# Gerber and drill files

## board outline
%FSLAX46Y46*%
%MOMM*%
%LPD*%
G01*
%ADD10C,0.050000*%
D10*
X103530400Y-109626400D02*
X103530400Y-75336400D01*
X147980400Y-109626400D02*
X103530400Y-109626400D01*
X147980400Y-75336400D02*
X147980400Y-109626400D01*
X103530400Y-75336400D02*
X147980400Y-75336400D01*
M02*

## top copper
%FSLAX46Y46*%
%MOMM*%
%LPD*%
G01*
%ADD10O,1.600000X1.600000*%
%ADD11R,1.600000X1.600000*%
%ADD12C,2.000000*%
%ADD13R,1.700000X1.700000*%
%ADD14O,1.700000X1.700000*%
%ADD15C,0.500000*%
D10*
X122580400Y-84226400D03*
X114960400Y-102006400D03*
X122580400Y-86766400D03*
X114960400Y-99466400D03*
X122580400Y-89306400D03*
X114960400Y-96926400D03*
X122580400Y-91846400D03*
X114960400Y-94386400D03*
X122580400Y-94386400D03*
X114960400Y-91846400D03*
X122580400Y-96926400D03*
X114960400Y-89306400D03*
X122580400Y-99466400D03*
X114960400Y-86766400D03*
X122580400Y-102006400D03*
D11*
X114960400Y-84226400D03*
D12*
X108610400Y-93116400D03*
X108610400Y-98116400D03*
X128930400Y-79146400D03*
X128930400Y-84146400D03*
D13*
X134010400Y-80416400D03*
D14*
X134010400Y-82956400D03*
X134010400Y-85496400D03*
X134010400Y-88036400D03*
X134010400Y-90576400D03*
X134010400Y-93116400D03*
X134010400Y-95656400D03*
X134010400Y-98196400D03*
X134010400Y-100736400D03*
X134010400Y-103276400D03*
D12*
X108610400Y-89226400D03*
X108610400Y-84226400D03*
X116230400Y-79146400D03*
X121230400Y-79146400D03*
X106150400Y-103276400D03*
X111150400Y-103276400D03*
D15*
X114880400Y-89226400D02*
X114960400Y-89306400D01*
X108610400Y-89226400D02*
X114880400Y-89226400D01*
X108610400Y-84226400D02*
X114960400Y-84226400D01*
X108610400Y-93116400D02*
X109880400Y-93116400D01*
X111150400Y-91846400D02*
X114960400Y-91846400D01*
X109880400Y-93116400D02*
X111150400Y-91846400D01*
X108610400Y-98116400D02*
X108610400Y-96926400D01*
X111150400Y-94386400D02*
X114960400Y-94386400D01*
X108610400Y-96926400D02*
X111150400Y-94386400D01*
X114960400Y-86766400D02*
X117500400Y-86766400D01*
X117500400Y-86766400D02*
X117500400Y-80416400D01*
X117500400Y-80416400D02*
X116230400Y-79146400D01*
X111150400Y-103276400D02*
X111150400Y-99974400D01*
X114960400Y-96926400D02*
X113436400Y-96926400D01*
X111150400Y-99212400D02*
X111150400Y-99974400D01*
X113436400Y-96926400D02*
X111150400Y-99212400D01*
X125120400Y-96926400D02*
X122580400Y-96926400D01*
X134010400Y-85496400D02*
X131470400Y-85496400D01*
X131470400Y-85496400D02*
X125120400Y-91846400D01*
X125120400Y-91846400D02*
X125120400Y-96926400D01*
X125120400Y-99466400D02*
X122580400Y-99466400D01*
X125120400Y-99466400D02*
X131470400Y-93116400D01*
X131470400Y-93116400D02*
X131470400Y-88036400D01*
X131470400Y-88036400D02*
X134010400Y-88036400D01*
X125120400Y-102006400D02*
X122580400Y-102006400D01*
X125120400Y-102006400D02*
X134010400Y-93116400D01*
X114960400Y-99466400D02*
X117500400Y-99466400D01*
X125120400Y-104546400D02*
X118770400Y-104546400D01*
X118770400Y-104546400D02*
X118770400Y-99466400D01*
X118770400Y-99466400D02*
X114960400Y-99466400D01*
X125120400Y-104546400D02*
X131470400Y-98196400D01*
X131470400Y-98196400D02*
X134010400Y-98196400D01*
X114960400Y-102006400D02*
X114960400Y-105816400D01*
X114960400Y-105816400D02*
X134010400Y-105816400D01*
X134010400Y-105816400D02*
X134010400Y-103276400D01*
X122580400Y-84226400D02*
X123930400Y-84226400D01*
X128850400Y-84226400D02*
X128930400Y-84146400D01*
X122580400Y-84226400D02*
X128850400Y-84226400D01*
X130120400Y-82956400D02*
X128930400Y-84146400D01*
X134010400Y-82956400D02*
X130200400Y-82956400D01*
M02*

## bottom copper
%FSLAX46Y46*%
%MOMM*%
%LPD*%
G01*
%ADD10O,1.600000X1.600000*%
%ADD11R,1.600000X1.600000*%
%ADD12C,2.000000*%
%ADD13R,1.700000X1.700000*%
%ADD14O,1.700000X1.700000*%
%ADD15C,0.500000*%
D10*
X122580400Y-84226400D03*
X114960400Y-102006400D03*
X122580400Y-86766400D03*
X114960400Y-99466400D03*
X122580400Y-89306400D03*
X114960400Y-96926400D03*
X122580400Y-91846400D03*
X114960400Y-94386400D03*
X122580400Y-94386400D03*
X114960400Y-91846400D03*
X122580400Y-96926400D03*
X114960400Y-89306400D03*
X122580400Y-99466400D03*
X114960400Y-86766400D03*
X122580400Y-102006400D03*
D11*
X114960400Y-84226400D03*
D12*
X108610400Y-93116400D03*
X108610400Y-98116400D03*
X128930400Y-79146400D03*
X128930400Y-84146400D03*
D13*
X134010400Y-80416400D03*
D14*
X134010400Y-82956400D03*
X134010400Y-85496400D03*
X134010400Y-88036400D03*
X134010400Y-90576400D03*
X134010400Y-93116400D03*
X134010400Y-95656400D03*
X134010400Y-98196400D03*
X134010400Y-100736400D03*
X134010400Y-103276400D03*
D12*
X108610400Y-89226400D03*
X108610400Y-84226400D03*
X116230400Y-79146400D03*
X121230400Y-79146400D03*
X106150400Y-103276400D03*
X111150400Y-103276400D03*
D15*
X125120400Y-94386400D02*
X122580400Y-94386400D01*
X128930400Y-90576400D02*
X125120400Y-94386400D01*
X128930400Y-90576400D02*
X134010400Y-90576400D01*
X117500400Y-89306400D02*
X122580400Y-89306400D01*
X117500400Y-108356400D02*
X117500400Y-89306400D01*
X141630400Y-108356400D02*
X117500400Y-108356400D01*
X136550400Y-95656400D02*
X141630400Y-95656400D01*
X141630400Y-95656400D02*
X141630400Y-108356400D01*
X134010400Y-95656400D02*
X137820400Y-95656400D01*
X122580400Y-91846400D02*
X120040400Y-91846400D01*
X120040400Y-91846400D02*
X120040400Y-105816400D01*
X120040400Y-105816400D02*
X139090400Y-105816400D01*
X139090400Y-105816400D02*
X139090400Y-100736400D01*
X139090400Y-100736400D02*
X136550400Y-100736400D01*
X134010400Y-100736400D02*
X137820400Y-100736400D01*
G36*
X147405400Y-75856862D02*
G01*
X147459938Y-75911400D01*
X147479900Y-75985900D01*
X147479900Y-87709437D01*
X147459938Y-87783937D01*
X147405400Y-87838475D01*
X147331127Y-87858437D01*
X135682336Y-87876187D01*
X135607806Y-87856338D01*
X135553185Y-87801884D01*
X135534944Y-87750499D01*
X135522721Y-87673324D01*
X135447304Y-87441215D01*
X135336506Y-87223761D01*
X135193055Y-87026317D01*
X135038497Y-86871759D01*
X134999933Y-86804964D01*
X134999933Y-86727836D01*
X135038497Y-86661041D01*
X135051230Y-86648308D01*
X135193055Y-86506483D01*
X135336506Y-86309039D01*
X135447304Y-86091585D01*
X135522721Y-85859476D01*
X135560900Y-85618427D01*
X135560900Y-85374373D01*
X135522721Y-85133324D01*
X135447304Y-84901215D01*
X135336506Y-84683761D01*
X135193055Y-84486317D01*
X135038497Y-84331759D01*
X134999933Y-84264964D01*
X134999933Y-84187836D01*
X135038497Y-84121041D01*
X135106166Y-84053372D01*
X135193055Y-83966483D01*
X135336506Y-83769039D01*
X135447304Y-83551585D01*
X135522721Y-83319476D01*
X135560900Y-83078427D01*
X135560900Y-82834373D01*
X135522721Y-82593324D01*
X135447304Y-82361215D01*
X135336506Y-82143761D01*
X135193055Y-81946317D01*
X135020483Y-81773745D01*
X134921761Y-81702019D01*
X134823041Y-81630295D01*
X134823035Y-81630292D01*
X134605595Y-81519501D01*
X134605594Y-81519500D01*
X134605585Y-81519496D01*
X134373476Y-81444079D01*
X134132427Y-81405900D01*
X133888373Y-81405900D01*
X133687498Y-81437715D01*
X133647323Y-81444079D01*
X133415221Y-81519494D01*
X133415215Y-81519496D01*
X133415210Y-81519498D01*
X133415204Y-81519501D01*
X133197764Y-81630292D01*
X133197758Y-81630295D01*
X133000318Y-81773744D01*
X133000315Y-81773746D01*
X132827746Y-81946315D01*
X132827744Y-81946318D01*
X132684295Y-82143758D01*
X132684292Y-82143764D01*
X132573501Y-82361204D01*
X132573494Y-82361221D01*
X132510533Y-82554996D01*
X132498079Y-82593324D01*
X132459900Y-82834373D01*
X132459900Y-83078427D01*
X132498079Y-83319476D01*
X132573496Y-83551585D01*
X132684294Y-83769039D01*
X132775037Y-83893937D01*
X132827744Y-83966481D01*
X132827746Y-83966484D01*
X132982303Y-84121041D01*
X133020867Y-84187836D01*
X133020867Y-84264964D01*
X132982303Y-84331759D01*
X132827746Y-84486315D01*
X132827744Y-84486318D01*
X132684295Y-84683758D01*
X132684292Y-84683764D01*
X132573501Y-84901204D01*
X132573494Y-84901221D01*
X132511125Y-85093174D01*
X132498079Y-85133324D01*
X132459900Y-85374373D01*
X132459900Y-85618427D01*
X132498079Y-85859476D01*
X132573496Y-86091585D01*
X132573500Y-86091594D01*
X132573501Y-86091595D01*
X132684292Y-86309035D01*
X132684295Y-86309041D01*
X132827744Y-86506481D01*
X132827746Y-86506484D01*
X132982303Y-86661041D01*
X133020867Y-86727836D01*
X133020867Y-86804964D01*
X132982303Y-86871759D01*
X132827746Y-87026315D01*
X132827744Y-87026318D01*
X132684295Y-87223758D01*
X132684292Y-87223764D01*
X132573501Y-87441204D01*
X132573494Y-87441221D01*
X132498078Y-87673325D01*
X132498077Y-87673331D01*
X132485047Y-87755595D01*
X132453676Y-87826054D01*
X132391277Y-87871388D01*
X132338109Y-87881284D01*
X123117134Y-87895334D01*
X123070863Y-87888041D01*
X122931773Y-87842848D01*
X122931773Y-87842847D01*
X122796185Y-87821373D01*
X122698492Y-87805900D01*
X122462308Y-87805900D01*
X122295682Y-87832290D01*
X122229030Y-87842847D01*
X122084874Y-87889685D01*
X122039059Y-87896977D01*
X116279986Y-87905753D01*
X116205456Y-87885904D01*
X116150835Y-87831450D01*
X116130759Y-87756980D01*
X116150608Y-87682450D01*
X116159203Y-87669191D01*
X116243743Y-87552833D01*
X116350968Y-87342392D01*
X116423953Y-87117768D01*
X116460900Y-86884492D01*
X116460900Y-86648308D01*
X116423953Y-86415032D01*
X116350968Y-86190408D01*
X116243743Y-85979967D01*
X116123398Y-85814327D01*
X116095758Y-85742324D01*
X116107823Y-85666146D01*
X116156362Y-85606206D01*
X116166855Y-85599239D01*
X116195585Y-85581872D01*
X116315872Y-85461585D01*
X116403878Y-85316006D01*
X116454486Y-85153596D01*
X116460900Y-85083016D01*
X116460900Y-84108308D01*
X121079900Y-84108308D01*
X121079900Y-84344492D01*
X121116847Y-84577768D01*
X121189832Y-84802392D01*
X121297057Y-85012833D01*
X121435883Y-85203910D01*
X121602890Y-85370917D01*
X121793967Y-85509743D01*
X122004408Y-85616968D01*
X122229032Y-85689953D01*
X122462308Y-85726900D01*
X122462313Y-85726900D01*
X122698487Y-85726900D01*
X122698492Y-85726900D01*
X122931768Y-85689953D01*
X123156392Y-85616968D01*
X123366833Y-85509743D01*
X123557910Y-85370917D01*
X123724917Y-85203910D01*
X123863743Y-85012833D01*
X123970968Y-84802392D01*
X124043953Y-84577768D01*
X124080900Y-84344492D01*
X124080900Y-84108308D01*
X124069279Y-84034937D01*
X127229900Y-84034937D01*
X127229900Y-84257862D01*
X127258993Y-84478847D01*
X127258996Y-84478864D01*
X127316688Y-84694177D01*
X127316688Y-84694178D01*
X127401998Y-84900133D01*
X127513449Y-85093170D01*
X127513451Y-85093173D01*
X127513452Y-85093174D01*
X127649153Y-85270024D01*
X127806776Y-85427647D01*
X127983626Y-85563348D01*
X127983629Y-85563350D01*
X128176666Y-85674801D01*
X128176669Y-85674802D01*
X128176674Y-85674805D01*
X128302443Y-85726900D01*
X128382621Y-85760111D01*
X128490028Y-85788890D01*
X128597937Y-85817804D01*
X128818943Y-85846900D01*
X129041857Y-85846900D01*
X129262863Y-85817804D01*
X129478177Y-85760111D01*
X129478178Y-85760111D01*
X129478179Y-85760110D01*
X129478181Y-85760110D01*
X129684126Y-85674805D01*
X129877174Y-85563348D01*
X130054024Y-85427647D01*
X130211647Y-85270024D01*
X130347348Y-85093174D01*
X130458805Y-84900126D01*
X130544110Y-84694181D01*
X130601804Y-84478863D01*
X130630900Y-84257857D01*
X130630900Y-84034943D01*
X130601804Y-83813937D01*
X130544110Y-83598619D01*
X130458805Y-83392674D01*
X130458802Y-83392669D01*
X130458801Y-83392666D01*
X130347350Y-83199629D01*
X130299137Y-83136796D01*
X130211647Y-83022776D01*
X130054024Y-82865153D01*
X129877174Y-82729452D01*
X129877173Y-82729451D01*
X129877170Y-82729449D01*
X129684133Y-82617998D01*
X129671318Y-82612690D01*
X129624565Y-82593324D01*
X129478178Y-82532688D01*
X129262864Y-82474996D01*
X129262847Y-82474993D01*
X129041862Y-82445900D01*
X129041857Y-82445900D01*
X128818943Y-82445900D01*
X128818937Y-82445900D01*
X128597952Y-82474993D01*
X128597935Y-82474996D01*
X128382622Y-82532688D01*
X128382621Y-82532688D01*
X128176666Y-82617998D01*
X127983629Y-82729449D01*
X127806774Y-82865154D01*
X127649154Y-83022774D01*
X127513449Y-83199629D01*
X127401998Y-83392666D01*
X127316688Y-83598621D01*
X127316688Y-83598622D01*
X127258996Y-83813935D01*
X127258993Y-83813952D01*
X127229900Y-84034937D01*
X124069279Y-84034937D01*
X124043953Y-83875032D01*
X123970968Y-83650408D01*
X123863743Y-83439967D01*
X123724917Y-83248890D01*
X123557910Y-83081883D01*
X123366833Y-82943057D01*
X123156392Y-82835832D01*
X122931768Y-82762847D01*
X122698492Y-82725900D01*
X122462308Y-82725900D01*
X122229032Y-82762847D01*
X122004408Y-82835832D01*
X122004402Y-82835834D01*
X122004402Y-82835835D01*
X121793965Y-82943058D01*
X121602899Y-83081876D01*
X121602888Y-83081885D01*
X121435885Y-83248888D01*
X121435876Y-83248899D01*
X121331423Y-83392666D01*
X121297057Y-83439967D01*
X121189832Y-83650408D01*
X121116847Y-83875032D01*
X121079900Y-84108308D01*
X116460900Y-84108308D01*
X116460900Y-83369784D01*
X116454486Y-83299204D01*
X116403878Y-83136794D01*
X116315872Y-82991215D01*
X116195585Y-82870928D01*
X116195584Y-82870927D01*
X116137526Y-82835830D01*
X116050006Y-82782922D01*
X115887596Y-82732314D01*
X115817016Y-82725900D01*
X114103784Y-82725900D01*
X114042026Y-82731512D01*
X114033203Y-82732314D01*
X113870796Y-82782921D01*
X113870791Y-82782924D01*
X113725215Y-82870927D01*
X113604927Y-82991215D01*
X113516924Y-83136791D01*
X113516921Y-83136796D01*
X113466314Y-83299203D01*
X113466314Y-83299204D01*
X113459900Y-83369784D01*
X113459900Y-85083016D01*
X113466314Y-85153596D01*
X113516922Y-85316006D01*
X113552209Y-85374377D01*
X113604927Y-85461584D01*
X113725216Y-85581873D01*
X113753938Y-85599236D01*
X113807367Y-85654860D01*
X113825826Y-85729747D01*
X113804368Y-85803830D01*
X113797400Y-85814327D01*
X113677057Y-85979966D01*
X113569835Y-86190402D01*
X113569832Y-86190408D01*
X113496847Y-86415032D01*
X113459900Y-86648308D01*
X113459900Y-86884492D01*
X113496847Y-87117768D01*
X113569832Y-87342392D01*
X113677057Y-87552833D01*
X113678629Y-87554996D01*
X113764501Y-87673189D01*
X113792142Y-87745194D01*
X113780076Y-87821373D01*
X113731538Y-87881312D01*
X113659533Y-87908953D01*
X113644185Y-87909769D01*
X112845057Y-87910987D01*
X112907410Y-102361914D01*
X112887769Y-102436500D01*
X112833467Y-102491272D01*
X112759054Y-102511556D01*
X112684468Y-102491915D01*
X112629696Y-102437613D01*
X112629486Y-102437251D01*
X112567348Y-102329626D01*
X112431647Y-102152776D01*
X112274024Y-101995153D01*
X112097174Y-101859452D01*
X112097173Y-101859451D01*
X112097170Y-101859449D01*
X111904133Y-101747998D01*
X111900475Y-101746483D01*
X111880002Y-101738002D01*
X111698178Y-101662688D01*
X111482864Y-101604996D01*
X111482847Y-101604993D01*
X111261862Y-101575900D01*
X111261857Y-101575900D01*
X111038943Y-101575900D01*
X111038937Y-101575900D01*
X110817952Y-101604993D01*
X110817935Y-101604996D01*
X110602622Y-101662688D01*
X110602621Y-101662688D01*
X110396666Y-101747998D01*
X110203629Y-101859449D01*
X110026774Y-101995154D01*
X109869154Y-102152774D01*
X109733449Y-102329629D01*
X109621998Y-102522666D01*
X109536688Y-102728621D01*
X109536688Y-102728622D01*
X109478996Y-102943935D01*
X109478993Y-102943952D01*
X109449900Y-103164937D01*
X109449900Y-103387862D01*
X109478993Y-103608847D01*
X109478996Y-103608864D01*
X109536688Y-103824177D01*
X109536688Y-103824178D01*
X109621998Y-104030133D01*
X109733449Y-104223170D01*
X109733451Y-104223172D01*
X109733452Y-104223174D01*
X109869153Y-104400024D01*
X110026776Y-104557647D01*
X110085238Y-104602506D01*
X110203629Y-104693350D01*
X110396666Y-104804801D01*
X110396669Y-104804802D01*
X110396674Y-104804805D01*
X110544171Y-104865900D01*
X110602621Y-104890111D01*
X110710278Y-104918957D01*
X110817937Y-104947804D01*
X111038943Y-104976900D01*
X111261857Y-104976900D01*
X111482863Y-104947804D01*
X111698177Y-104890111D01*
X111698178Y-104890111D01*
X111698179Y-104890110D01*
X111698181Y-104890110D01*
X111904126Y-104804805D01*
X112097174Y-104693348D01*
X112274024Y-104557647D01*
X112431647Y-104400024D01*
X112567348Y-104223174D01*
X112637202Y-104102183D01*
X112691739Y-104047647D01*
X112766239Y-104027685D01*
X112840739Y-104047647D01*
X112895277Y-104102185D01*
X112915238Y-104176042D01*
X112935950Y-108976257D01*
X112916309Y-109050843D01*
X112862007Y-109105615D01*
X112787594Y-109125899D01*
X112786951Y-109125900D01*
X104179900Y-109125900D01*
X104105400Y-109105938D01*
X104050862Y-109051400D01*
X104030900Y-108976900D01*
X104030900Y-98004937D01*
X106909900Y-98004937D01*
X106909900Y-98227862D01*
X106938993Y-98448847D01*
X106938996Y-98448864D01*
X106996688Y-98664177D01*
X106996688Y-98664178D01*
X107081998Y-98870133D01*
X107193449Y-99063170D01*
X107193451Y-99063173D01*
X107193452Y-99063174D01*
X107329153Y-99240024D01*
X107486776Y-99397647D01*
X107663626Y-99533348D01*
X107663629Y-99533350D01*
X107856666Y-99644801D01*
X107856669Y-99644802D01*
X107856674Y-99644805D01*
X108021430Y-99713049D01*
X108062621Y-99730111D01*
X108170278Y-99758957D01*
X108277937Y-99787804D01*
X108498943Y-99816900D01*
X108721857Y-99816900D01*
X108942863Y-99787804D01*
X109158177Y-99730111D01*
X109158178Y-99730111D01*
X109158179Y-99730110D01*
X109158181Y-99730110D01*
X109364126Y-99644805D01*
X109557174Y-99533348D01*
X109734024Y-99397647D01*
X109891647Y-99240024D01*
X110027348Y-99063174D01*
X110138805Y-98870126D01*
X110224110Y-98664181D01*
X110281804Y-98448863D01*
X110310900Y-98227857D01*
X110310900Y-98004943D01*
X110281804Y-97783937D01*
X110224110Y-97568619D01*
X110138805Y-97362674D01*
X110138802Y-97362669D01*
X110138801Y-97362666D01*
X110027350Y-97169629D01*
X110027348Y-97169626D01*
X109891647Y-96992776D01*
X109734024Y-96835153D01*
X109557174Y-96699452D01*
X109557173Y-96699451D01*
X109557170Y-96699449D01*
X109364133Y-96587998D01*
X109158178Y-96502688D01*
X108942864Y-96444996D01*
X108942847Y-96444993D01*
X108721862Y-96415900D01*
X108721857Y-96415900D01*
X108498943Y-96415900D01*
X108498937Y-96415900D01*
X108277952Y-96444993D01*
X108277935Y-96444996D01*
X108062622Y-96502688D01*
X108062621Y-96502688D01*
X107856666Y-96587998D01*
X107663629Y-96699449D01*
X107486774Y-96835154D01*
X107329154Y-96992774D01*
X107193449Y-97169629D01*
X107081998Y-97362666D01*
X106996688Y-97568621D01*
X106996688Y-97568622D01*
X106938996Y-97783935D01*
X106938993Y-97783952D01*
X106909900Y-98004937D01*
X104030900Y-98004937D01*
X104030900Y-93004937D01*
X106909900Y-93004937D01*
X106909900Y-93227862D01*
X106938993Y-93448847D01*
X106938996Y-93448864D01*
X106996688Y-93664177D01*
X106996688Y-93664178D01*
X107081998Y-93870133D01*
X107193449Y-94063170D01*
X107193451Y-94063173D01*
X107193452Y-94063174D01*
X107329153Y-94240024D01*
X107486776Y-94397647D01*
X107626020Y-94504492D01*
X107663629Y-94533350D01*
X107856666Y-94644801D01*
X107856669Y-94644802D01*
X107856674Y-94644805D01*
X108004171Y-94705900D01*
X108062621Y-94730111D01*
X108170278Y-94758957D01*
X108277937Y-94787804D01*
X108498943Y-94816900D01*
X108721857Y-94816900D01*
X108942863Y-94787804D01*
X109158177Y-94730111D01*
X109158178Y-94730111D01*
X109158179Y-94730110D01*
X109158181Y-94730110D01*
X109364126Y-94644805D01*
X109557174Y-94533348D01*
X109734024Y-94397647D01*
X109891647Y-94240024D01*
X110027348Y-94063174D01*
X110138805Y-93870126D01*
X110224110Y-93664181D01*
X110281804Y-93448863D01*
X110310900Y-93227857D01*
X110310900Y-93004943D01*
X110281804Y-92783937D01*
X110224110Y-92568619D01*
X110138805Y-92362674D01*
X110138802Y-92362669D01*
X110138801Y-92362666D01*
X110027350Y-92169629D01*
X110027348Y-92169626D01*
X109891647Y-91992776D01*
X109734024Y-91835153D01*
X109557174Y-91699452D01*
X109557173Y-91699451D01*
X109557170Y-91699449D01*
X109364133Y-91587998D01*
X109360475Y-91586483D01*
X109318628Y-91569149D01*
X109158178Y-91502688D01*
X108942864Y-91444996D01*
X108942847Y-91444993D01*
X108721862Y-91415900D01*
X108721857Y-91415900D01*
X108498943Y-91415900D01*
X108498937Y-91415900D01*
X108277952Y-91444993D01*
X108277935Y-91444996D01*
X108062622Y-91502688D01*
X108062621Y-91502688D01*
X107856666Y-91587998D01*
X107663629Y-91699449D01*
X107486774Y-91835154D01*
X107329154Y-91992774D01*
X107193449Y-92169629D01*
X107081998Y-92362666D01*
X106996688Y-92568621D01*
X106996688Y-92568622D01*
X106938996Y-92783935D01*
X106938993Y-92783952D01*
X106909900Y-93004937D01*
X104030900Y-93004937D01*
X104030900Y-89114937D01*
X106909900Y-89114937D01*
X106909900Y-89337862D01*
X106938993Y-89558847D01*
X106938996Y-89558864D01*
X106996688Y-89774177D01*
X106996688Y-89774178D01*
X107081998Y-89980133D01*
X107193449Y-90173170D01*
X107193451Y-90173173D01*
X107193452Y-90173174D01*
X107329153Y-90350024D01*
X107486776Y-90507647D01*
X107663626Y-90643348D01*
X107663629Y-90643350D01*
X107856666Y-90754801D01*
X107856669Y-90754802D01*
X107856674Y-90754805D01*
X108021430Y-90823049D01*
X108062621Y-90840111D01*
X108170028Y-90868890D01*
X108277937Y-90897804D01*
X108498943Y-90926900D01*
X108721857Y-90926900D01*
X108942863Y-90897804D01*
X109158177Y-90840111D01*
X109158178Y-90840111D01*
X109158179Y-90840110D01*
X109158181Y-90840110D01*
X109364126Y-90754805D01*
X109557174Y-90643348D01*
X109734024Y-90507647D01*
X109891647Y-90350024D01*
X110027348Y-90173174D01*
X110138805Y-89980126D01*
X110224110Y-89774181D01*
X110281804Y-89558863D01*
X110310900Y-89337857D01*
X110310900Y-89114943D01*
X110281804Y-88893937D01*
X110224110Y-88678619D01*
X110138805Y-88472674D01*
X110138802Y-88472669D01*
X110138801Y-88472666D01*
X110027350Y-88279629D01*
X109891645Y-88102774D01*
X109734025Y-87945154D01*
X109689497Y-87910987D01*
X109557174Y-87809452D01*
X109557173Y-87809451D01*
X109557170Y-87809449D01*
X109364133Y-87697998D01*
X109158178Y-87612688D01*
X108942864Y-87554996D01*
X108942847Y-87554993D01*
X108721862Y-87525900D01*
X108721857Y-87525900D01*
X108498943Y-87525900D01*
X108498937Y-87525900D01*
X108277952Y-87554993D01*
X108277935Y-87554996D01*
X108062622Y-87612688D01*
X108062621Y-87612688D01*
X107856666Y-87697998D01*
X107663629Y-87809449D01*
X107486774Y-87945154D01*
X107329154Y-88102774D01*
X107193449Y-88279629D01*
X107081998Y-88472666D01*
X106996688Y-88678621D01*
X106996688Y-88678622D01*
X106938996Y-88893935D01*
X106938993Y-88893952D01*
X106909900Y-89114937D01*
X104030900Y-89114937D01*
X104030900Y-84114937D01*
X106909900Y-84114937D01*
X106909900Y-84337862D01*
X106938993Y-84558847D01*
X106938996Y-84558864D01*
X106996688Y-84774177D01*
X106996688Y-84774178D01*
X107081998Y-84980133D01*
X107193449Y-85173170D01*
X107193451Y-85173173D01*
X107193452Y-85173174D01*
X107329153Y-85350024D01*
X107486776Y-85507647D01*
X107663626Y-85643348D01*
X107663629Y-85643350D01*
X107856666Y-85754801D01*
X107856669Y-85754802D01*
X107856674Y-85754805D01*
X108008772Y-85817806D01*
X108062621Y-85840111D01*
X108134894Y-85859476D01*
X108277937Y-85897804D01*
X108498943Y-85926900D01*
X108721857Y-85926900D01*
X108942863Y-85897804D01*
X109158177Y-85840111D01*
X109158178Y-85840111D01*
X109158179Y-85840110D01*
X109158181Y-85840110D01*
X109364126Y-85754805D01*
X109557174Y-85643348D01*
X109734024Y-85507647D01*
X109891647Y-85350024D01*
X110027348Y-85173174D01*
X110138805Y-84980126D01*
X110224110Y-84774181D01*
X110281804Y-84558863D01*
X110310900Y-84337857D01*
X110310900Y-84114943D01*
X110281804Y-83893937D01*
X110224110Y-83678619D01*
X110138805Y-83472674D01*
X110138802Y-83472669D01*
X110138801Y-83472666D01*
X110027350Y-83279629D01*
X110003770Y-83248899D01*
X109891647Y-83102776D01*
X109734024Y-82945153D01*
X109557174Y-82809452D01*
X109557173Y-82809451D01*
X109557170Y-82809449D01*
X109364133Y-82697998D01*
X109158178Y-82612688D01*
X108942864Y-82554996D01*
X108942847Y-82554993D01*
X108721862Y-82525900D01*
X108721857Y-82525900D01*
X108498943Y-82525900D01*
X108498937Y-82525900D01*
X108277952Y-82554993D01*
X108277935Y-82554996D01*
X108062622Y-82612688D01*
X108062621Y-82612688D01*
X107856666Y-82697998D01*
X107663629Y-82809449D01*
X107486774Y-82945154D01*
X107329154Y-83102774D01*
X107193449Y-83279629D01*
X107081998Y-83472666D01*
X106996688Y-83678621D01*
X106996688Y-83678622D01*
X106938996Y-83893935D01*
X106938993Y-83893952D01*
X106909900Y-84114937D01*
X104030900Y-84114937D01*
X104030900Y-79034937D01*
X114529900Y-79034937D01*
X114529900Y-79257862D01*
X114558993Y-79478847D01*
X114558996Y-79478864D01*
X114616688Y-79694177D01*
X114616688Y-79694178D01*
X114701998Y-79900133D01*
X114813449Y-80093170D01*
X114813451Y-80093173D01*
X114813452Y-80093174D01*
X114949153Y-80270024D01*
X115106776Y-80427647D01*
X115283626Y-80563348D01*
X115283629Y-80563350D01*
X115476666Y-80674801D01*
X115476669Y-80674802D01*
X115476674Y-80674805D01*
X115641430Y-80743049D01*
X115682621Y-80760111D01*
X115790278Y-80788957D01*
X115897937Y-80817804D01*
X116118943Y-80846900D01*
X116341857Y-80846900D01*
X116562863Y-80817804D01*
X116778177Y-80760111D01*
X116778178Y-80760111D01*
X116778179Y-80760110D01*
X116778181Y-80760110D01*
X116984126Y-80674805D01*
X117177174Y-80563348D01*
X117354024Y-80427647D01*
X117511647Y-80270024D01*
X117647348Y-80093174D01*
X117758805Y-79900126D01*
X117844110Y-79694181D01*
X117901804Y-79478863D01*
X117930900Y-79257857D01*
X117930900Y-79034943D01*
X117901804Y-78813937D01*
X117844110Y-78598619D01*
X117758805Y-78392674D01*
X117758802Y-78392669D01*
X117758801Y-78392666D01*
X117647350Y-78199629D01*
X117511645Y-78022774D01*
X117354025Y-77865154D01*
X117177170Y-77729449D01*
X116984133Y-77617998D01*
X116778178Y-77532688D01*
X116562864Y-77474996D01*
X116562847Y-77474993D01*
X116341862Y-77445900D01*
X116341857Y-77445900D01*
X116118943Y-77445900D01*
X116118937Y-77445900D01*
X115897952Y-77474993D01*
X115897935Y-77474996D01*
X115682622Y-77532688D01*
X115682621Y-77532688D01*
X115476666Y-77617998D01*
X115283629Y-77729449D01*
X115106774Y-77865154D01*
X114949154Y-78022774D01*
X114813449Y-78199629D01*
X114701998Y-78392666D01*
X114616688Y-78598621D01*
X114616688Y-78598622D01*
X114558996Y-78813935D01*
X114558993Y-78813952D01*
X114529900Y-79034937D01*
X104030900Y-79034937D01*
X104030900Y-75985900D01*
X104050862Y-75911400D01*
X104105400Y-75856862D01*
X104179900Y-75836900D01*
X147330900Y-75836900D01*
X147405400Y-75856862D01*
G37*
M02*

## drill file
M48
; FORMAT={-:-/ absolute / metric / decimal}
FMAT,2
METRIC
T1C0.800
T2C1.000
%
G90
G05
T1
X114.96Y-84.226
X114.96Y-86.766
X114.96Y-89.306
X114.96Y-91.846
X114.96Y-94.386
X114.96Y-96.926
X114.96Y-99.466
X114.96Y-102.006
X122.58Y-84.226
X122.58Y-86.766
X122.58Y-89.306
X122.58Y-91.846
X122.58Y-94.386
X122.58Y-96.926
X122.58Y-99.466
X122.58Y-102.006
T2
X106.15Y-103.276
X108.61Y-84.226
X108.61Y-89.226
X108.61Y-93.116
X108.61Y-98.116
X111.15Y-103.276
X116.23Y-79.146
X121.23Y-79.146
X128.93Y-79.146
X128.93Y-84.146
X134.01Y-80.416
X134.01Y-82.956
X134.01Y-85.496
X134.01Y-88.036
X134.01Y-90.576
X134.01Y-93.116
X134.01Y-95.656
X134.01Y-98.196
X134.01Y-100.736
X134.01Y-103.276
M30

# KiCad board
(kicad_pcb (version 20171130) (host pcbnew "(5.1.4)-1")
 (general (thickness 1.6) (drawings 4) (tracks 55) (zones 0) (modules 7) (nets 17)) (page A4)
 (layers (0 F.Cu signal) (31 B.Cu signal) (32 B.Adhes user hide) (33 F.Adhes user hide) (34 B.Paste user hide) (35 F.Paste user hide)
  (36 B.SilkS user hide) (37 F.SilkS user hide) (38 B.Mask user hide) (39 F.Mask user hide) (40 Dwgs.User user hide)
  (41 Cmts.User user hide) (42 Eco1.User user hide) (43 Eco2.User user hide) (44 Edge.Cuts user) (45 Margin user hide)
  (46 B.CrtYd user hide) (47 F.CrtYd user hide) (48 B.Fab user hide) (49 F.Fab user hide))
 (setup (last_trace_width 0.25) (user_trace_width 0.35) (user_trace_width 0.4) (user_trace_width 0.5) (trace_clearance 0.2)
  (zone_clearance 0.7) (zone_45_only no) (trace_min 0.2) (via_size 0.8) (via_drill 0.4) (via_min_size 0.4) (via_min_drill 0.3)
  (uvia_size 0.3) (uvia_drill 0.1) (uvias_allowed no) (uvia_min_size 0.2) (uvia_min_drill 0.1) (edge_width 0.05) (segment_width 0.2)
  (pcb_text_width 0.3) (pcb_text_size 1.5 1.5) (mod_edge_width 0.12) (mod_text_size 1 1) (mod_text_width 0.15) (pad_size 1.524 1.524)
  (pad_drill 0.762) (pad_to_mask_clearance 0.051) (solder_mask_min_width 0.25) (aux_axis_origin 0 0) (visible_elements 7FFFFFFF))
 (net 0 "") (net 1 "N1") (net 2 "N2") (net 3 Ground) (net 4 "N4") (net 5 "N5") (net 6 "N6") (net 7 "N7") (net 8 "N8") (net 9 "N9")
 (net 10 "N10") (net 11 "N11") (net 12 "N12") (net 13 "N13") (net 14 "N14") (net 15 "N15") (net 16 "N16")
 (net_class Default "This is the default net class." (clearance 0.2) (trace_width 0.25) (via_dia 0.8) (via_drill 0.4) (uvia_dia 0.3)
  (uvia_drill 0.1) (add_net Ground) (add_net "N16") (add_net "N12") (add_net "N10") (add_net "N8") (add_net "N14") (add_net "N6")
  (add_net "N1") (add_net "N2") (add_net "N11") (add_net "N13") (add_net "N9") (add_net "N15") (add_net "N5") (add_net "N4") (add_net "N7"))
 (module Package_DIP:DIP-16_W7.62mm (layer F.Cu) (at 114.9604 84.2264)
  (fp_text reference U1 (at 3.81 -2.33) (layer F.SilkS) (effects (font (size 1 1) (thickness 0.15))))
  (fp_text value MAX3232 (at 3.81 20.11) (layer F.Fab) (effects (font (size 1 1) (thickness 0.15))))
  (pad 16 thru_hole oval (at 7.62 0) (size 1.6 1.6) (drill 0.8) (layers *.Cu *.Mask) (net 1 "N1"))
  (pad 8 thru_hole oval (at 0 17.78) (size 1.6 1.6) (drill 0.8) (layers *.Cu *.Mask) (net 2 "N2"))
  (pad 15 thru_hole oval (at 7.62 2.54) (size 1.6 1.6) (drill 0.8) (layers *.Cu *.Mask) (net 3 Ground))
  (pad 7 thru_hole oval (at 0 15.24) (size 1.6 1.6) (drill 0.8) (layers *.Cu *.Mask) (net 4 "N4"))
  (pad 14 thru_hole oval (at 7.62 5.08) (size 1.6 1.6) (drill 0.8) (layers *.Cu *.Mask) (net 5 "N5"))
  (pad 6 thru_hole oval (at 0 12.7) (size 1.6 1.6) (drill 0.8) (layers *.Cu *.Mask) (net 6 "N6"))
  (pad 13 thru_hole oval (at 7.62 7.62) (size 1.6 1.6) (drill 0.8) (layers *.Cu *.Mask) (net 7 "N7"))
  (pad 5 thru_hole oval (at 0 10.16) (size 1.6 1.6) (drill 0.8) (layers *.Cu *.Mask) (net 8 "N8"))
  (pad 12 thru_hole oval (at 7.62 10.16) (size 1.6 1.6) (drill 0.8) (layers *.Cu *.Mask) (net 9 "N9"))
  (pad 4 thru_hole oval (at 0 7.62) (size 1.6 1.6) (drill 0.8) (layers *.Cu *.Mask) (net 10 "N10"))
  (pad 11 thru_hole oval (at 7.62 12.7) (size 1.6 1.6) (drill 0.8) (layers *.Cu *.Mask) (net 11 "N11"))
  (pad 3 thru_hole oval (at 0 5.08) (size 1.6 1.6) (drill 0.8) (layers *.Cu *.Mask) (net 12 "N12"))
  (pad 10 thru_hole oval (at 7.62 15.24) (size 1.6 1.6) (drill 0.8) (layers *.Cu *.Mask) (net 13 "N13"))
  (pad 2 thru_hole oval (at 0 2.54) (size 1.6 1.6) (drill 0.8) (layers *.Cu *.Mask) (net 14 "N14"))
  (pad 9 thru_hole oval (at 7.62 17.78) (size 1.6 1.6) (drill 0.8) (layers *.Cu *.Mask) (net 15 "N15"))
  (pad 1 thru_hole rect (at 0 0) (size 1.6 1.6) (drill 0.8) (layers *.Cu *.Mask) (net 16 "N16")))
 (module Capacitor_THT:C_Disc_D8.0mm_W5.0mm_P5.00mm (layer F.Cu) (at 108.6104 93.1164 270)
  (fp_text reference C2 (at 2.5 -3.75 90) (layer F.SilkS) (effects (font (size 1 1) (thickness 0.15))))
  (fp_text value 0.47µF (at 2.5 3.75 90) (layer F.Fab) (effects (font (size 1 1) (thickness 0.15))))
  (pad 1 thru_hole circle (at 0 0 270) (size 2 2) (drill 1) (layers *.Cu *.Mask) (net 10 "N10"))
  (pad 2 thru_hole circle (at 5 0 270) (size 2 2) (drill 1) (layers *.Cu *.Mask) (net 8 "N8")))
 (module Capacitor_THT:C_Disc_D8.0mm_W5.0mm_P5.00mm (layer F.Cu) (at 128.9304 79.1464 270)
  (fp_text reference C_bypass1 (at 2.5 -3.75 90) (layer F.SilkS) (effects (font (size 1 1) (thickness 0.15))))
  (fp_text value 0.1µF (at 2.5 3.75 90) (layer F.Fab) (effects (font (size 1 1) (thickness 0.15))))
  (pad 1 thru_hole circle (at 0 0 270) (size 2 2) (drill 1) (layers *.Cu *.Mask) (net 3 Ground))
  (pad 2 thru_hole circle (at 5 0 270) (size 2 2) (drill 1) (layers *.Cu *.Mask) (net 1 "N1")))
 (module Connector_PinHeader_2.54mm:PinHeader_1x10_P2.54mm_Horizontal (layer F.Cu) (at 134.0104 80.4164)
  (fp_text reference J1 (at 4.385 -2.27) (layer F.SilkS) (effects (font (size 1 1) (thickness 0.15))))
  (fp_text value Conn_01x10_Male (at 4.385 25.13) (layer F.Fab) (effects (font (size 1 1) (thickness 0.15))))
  (pad 1 thru_hole rect (at 0 0) (size 1.7 1.7) (drill 1) (layers *.Cu *.Mask) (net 3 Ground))
  (pad 2 thru_hole oval (at 0 2.54) (size 1.7 1.7) (drill 1) (layers *.Cu *.Mask) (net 1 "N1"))
  (pad 3 thru_hole oval (at 0 5.08) (size 1.7 1.7) (drill 1) (layers *.Cu *.Mask) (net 11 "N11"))
  (pad 4 thru_hole oval (at 0 7.62) (size 1.7 1.7) (drill 1) (layers *.Cu *.Mask) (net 13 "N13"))
  (pad 5 thru_hole oval (at 0 10.16) (size 1.7 1.7) (drill 1) (layers *.Cu *.Mask) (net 9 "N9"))
  (pad 6 thru_hole oval (at 0 12.7) (size 1.7 1.7) (drill 1) (layers *.Cu *.Mask) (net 15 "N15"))
  (pad 7 thru_hole oval (at 0 15.24) (size 1.7 1.7) (drill 1) (layers *.Cu *.Mask) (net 5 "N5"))
  (pad 8 thru_hole oval (at 0 17.78) (size 1.7 1.7) (drill 1) (layers *.Cu *.Mask) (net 4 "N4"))
  (pad 9 thru_hole oval (at 0 20.32) (size 1.7 1.7) (drill 1) (layers *.Cu *.Mask) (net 7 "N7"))
  (pad 10 thru_hole oval (at 0 22.86) (size 1.7 1.7) (drill 1) (layers *.Cu *.Mask) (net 2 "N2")))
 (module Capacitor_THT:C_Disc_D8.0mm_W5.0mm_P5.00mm (layer F.Cu) (at 108.6104 84.2264 270)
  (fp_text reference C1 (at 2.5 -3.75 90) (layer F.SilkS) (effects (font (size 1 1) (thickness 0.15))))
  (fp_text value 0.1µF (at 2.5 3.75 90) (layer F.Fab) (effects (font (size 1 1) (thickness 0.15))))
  (pad 2 thru_hole circle (at 5 0 270) (size 2 2) (drill 1) (layers *.Cu *.Mask) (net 12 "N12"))
  (pad 1 thru_hole circle (at 0 0 270) (size 2 2) (drill 1) (layers *.Cu *.Mask) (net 16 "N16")))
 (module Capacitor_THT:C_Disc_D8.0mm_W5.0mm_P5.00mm (layer F.Cu) (at 116.2304 79.1464)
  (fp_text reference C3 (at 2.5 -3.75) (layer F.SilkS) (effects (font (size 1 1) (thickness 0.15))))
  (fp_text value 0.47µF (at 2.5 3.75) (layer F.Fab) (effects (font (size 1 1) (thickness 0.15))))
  (pad 1 thru_hole circle (at 0 0) (size 2 2) (drill 1) (layers *.Cu *.Mask) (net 14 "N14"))
  (pad 2 thru_hole circle (at 5 0) (size 2 2) (drill 1) (layers *.Cu *.Mask) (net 3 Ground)))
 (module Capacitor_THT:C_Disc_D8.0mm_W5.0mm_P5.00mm (layer F.Cu) (at 111.1504 103.2764 180)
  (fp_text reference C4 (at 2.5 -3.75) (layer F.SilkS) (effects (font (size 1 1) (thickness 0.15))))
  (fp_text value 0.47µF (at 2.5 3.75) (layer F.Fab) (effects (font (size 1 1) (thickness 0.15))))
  (pad 2 thru_hole circle (at 5 0 180) (size 2 2) (drill 1) (layers *.Cu *.Mask) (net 3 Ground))
  (pad 1 thru_hole circle (at 0 0 180) (size 2 2) (drill 1) (layers *.Cu *.Mask) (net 6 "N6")))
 (gr_line (start 103.5304 109.6264) (end 103.5304 75.3364) (layer Edge.Cuts) (width 0.05))
 (gr_line (start 147.9804 109.6264) (end 103.5304 109.6264) (layer Edge.Cuts) (width 0.05))
 (gr_line (start 147.9804 75.3364) (end 147.9804 109.6264) (layer Edge.Cuts) (width 0.05))
 (gr_line (start 103.5304 75.3364) (end 147.9804 75.3364) (layer Edge.Cuts) (width 0.05))
 (segment (start 114.8804 89.2264) (end 114.9604 89.3064) (width 0.5) (layer F.Cu) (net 12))
 (segment (start 108.6104 89.2264) (end 114.8804 89.2264) (width 0.5) (layer F.Cu) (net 12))
 (segment (start 108.6104 84.2264) (end 114.9604 84.2264) (width 0.5) (layer F.Cu) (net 16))
 (segment (start 108.6104 93.1164) (end 109.8804 93.1164) (width 0.5) (layer F.Cu) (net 10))
 (segment (start 111.1504 91.8464) (end 114.9604 91.8464) (width 0.5) (layer F.Cu) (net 10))
 (segment (start 109.8804 93.1164) (end 111.1504 91.8464) (width 0.5) (layer F.Cu) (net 10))
 (segment (start 108.6104 98.1164) (end 108.6104 96.9264) (width 0.5) (layer F.Cu) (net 8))
 (segment (start 111.1504 94.3864) (end 114.9604 94.3864) (width 0.5) (layer F.Cu) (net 8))
 (segment (start 108.6104 96.9264) (end 111.1504 94.3864) (width 0.5) (layer F.Cu) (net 8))
 (segment (start 114.9604 86.7664) (end 117.5004 86.7664) (width 0.5) (layer F.Cu) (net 14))
 (segment (start 117.5004 86.7664) (end 117.5004 80.4164) (width 0.5) (layer F.Cu) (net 14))
 (segment (start 117.5004 80.4164) (end 116.2304 79.1464) (width 0.5) (layer F.Cu) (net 14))
 (segment (start 111.1504 103.2764) (end 111.1504 99.9744) (width 0.5) (layer F.Cu) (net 6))
 (segment (start 114.9604 96.9264) (end 113.4364 96.9264) (width 0.5) (layer F.Cu) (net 6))
 (segment (start 111.1504 99.2124) (end 111.1504 99.9744) (width 0.5) (layer F.Cu) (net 6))
 (segment (start 113.4364 96.9264) (end 111.1504 99.2124) (width 0.5) (layer F.Cu) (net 6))
 (segment (start 125.1204 96.9264) (end 122.5804 96.9264) (width 0.5) (layer F.Cu) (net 11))
 (segment (start 134.0104 85.4964) (end 131.4704 85.4964) (width 0.5) (layer F.Cu) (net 11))
 (segment (start 131.4704 85.4964) (end 125.1204 91.8464) (width 0.5) (layer F.Cu) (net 11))
 (segment (start 125.1204 91.8464) (end 125.1204 96.9264) (width 0.5) (layer F.Cu) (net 11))
 (segment (start 125.1204 99.4664) (end 122.5804 99.4664) (width 0.5) (layer F.Cu) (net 13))
 (segment (start 125.1204 99.4664) (end 131.4704 93.1164) (width 0.5) (layer F.Cu) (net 13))
 (segment (start 131.4704 93.1164) (end 131.4704 88.0364) (width 0.5) (layer F.Cu) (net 13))
 (segment (start 131.4704 88.0364) (end 134.0104 88.0364) (width 0.5) (layer F.Cu) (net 13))
 (segment (start 125.1204 94.3864) (end 122.5804 94.3864) (width 0.5) (layer B.Cu) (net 9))
 (segment (start 128.9304 90.5764) (end 125.1204 94.3864) (width 0.5) (layer B.Cu) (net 9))
 (segment (start 128.9304 90.5764) (end 134.0104 90.5764) (width 0.5) (layer B.Cu) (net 9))
 (segment (start 125.1204 102.0064) (end 122.5804 102.0064) (width 0.5) (layer F.Cu) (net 15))
 (segment (start 125.1204 102.0064) (end 134.0104 93.1164) (width 0.5) (layer F.Cu) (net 15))
 (segment (start 117.5004 89.3064) (end 122.5804 89.3064) (width 0.5) (layer B.Cu) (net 5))
 (segment (start 117.5004 108.3564) (end 117.5004 89.3064) (width 0.5) (layer B.Cu) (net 5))
 (segment (start 141.6304 108.3564) (end 117.5004 108.3564) (width 0.5) (layer B.Cu) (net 5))
 (segment (start 136.5504 95.6564) (end 141.6304 95.6564) (width 0.5) (layer B.Cu) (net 5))
 (segment (start 141.6304 95.6564) (end 141.6304 108.3564) (width 0.5) (layer B.Cu) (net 5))
 (segment (start 134.0104 95.6564) (end 137.8204 95.6564) (width 0.5) (layer B.Cu) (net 5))
 (segment (start 114.9604 99.4664) (end 117.5004 99.4664) (width 0.5) (layer F.Cu) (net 4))
 (segment (start 125.1204 104.5464) (end 118.7704 104.5464) (width 0.5) (layer F.Cu) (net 4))
 (segment (start 118.7704 104.5464) (end 118.7704 99.4664) (width 0.5) (layer F.Cu) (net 4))
 (segment (start 118.7704 99.4664) (end 114.9604 99.4664) (width 0.5) (layer F.Cu) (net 4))
 (segment (start 125.1204 104.5464) (end 131.4704 98.1964) (width 0.5) (layer F.Cu) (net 4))
 (segment (start 131.4704 98.1964) (end 134.0104 98.1964) (width 0.5) (layer F.Cu) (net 4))
 (segment (start 122.5804 91.8464) (end 120.0404 91.8464) (width 0.5) (layer B.Cu) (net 7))
 (segment (start 120.0404 91.8464) (end 120.0404 105.8164) (width 0.5) (layer B.Cu) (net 7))
 (segment (start 120.0404 105.8164) (end 139.0904 105.8164) (width 0.5) (layer B.Cu) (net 7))
 (segment (start 139.0904 105.8164) (end 139.0904 100.7364) (width 0.5) (layer B.Cu) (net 7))
 (segment (start 139.0904 100.7364) (end 136.5504 100.7364) (width 0.5) (layer B.Cu) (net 7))
 (segment (start 134.0104 100.7364) (end 137.8204 100.7364) (width 0.5) (layer B.Cu) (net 7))
 (segment (start 114.9604 102.0064) (end 114.9604 105.8164) (width 0.5) (layer F.Cu) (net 2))
 (segment (start 114.9604 105.8164) (end 134.0104 105.8164) (width 0.5) (layer F.Cu) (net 2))
 (segment (start 134.0104 105.8164) (end 134.0104 103.2764) (width 0.5) (layer F.Cu) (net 2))
 (segment (start 122.5804 84.2264) (end 123.9304 84.2264) (width 0.5) (layer F.Cu) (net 1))
 (segment (start 128.8504 84.2264) (end 128.9304 84.1464) (width 0.5) (layer F.Cu) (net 1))
 (segment (start 122.5804 84.2264) (end 128.8504 84.2264) (width 0.5) (layer F.Cu) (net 1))
 (segment (start 130.1204 82.9564) (end 128.9304 84.1464) (width 0.5) (layer F.Cu) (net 1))
 (segment (start 134.0104 82.9564) (end 130.2004 82.9564) (width 0.5) (layer F.Cu) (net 1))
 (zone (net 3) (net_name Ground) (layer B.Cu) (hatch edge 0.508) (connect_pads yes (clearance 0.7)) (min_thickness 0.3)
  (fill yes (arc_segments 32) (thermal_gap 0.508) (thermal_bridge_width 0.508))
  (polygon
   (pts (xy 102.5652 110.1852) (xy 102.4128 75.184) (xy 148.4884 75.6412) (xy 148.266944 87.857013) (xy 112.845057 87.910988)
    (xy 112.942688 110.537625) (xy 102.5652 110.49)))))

